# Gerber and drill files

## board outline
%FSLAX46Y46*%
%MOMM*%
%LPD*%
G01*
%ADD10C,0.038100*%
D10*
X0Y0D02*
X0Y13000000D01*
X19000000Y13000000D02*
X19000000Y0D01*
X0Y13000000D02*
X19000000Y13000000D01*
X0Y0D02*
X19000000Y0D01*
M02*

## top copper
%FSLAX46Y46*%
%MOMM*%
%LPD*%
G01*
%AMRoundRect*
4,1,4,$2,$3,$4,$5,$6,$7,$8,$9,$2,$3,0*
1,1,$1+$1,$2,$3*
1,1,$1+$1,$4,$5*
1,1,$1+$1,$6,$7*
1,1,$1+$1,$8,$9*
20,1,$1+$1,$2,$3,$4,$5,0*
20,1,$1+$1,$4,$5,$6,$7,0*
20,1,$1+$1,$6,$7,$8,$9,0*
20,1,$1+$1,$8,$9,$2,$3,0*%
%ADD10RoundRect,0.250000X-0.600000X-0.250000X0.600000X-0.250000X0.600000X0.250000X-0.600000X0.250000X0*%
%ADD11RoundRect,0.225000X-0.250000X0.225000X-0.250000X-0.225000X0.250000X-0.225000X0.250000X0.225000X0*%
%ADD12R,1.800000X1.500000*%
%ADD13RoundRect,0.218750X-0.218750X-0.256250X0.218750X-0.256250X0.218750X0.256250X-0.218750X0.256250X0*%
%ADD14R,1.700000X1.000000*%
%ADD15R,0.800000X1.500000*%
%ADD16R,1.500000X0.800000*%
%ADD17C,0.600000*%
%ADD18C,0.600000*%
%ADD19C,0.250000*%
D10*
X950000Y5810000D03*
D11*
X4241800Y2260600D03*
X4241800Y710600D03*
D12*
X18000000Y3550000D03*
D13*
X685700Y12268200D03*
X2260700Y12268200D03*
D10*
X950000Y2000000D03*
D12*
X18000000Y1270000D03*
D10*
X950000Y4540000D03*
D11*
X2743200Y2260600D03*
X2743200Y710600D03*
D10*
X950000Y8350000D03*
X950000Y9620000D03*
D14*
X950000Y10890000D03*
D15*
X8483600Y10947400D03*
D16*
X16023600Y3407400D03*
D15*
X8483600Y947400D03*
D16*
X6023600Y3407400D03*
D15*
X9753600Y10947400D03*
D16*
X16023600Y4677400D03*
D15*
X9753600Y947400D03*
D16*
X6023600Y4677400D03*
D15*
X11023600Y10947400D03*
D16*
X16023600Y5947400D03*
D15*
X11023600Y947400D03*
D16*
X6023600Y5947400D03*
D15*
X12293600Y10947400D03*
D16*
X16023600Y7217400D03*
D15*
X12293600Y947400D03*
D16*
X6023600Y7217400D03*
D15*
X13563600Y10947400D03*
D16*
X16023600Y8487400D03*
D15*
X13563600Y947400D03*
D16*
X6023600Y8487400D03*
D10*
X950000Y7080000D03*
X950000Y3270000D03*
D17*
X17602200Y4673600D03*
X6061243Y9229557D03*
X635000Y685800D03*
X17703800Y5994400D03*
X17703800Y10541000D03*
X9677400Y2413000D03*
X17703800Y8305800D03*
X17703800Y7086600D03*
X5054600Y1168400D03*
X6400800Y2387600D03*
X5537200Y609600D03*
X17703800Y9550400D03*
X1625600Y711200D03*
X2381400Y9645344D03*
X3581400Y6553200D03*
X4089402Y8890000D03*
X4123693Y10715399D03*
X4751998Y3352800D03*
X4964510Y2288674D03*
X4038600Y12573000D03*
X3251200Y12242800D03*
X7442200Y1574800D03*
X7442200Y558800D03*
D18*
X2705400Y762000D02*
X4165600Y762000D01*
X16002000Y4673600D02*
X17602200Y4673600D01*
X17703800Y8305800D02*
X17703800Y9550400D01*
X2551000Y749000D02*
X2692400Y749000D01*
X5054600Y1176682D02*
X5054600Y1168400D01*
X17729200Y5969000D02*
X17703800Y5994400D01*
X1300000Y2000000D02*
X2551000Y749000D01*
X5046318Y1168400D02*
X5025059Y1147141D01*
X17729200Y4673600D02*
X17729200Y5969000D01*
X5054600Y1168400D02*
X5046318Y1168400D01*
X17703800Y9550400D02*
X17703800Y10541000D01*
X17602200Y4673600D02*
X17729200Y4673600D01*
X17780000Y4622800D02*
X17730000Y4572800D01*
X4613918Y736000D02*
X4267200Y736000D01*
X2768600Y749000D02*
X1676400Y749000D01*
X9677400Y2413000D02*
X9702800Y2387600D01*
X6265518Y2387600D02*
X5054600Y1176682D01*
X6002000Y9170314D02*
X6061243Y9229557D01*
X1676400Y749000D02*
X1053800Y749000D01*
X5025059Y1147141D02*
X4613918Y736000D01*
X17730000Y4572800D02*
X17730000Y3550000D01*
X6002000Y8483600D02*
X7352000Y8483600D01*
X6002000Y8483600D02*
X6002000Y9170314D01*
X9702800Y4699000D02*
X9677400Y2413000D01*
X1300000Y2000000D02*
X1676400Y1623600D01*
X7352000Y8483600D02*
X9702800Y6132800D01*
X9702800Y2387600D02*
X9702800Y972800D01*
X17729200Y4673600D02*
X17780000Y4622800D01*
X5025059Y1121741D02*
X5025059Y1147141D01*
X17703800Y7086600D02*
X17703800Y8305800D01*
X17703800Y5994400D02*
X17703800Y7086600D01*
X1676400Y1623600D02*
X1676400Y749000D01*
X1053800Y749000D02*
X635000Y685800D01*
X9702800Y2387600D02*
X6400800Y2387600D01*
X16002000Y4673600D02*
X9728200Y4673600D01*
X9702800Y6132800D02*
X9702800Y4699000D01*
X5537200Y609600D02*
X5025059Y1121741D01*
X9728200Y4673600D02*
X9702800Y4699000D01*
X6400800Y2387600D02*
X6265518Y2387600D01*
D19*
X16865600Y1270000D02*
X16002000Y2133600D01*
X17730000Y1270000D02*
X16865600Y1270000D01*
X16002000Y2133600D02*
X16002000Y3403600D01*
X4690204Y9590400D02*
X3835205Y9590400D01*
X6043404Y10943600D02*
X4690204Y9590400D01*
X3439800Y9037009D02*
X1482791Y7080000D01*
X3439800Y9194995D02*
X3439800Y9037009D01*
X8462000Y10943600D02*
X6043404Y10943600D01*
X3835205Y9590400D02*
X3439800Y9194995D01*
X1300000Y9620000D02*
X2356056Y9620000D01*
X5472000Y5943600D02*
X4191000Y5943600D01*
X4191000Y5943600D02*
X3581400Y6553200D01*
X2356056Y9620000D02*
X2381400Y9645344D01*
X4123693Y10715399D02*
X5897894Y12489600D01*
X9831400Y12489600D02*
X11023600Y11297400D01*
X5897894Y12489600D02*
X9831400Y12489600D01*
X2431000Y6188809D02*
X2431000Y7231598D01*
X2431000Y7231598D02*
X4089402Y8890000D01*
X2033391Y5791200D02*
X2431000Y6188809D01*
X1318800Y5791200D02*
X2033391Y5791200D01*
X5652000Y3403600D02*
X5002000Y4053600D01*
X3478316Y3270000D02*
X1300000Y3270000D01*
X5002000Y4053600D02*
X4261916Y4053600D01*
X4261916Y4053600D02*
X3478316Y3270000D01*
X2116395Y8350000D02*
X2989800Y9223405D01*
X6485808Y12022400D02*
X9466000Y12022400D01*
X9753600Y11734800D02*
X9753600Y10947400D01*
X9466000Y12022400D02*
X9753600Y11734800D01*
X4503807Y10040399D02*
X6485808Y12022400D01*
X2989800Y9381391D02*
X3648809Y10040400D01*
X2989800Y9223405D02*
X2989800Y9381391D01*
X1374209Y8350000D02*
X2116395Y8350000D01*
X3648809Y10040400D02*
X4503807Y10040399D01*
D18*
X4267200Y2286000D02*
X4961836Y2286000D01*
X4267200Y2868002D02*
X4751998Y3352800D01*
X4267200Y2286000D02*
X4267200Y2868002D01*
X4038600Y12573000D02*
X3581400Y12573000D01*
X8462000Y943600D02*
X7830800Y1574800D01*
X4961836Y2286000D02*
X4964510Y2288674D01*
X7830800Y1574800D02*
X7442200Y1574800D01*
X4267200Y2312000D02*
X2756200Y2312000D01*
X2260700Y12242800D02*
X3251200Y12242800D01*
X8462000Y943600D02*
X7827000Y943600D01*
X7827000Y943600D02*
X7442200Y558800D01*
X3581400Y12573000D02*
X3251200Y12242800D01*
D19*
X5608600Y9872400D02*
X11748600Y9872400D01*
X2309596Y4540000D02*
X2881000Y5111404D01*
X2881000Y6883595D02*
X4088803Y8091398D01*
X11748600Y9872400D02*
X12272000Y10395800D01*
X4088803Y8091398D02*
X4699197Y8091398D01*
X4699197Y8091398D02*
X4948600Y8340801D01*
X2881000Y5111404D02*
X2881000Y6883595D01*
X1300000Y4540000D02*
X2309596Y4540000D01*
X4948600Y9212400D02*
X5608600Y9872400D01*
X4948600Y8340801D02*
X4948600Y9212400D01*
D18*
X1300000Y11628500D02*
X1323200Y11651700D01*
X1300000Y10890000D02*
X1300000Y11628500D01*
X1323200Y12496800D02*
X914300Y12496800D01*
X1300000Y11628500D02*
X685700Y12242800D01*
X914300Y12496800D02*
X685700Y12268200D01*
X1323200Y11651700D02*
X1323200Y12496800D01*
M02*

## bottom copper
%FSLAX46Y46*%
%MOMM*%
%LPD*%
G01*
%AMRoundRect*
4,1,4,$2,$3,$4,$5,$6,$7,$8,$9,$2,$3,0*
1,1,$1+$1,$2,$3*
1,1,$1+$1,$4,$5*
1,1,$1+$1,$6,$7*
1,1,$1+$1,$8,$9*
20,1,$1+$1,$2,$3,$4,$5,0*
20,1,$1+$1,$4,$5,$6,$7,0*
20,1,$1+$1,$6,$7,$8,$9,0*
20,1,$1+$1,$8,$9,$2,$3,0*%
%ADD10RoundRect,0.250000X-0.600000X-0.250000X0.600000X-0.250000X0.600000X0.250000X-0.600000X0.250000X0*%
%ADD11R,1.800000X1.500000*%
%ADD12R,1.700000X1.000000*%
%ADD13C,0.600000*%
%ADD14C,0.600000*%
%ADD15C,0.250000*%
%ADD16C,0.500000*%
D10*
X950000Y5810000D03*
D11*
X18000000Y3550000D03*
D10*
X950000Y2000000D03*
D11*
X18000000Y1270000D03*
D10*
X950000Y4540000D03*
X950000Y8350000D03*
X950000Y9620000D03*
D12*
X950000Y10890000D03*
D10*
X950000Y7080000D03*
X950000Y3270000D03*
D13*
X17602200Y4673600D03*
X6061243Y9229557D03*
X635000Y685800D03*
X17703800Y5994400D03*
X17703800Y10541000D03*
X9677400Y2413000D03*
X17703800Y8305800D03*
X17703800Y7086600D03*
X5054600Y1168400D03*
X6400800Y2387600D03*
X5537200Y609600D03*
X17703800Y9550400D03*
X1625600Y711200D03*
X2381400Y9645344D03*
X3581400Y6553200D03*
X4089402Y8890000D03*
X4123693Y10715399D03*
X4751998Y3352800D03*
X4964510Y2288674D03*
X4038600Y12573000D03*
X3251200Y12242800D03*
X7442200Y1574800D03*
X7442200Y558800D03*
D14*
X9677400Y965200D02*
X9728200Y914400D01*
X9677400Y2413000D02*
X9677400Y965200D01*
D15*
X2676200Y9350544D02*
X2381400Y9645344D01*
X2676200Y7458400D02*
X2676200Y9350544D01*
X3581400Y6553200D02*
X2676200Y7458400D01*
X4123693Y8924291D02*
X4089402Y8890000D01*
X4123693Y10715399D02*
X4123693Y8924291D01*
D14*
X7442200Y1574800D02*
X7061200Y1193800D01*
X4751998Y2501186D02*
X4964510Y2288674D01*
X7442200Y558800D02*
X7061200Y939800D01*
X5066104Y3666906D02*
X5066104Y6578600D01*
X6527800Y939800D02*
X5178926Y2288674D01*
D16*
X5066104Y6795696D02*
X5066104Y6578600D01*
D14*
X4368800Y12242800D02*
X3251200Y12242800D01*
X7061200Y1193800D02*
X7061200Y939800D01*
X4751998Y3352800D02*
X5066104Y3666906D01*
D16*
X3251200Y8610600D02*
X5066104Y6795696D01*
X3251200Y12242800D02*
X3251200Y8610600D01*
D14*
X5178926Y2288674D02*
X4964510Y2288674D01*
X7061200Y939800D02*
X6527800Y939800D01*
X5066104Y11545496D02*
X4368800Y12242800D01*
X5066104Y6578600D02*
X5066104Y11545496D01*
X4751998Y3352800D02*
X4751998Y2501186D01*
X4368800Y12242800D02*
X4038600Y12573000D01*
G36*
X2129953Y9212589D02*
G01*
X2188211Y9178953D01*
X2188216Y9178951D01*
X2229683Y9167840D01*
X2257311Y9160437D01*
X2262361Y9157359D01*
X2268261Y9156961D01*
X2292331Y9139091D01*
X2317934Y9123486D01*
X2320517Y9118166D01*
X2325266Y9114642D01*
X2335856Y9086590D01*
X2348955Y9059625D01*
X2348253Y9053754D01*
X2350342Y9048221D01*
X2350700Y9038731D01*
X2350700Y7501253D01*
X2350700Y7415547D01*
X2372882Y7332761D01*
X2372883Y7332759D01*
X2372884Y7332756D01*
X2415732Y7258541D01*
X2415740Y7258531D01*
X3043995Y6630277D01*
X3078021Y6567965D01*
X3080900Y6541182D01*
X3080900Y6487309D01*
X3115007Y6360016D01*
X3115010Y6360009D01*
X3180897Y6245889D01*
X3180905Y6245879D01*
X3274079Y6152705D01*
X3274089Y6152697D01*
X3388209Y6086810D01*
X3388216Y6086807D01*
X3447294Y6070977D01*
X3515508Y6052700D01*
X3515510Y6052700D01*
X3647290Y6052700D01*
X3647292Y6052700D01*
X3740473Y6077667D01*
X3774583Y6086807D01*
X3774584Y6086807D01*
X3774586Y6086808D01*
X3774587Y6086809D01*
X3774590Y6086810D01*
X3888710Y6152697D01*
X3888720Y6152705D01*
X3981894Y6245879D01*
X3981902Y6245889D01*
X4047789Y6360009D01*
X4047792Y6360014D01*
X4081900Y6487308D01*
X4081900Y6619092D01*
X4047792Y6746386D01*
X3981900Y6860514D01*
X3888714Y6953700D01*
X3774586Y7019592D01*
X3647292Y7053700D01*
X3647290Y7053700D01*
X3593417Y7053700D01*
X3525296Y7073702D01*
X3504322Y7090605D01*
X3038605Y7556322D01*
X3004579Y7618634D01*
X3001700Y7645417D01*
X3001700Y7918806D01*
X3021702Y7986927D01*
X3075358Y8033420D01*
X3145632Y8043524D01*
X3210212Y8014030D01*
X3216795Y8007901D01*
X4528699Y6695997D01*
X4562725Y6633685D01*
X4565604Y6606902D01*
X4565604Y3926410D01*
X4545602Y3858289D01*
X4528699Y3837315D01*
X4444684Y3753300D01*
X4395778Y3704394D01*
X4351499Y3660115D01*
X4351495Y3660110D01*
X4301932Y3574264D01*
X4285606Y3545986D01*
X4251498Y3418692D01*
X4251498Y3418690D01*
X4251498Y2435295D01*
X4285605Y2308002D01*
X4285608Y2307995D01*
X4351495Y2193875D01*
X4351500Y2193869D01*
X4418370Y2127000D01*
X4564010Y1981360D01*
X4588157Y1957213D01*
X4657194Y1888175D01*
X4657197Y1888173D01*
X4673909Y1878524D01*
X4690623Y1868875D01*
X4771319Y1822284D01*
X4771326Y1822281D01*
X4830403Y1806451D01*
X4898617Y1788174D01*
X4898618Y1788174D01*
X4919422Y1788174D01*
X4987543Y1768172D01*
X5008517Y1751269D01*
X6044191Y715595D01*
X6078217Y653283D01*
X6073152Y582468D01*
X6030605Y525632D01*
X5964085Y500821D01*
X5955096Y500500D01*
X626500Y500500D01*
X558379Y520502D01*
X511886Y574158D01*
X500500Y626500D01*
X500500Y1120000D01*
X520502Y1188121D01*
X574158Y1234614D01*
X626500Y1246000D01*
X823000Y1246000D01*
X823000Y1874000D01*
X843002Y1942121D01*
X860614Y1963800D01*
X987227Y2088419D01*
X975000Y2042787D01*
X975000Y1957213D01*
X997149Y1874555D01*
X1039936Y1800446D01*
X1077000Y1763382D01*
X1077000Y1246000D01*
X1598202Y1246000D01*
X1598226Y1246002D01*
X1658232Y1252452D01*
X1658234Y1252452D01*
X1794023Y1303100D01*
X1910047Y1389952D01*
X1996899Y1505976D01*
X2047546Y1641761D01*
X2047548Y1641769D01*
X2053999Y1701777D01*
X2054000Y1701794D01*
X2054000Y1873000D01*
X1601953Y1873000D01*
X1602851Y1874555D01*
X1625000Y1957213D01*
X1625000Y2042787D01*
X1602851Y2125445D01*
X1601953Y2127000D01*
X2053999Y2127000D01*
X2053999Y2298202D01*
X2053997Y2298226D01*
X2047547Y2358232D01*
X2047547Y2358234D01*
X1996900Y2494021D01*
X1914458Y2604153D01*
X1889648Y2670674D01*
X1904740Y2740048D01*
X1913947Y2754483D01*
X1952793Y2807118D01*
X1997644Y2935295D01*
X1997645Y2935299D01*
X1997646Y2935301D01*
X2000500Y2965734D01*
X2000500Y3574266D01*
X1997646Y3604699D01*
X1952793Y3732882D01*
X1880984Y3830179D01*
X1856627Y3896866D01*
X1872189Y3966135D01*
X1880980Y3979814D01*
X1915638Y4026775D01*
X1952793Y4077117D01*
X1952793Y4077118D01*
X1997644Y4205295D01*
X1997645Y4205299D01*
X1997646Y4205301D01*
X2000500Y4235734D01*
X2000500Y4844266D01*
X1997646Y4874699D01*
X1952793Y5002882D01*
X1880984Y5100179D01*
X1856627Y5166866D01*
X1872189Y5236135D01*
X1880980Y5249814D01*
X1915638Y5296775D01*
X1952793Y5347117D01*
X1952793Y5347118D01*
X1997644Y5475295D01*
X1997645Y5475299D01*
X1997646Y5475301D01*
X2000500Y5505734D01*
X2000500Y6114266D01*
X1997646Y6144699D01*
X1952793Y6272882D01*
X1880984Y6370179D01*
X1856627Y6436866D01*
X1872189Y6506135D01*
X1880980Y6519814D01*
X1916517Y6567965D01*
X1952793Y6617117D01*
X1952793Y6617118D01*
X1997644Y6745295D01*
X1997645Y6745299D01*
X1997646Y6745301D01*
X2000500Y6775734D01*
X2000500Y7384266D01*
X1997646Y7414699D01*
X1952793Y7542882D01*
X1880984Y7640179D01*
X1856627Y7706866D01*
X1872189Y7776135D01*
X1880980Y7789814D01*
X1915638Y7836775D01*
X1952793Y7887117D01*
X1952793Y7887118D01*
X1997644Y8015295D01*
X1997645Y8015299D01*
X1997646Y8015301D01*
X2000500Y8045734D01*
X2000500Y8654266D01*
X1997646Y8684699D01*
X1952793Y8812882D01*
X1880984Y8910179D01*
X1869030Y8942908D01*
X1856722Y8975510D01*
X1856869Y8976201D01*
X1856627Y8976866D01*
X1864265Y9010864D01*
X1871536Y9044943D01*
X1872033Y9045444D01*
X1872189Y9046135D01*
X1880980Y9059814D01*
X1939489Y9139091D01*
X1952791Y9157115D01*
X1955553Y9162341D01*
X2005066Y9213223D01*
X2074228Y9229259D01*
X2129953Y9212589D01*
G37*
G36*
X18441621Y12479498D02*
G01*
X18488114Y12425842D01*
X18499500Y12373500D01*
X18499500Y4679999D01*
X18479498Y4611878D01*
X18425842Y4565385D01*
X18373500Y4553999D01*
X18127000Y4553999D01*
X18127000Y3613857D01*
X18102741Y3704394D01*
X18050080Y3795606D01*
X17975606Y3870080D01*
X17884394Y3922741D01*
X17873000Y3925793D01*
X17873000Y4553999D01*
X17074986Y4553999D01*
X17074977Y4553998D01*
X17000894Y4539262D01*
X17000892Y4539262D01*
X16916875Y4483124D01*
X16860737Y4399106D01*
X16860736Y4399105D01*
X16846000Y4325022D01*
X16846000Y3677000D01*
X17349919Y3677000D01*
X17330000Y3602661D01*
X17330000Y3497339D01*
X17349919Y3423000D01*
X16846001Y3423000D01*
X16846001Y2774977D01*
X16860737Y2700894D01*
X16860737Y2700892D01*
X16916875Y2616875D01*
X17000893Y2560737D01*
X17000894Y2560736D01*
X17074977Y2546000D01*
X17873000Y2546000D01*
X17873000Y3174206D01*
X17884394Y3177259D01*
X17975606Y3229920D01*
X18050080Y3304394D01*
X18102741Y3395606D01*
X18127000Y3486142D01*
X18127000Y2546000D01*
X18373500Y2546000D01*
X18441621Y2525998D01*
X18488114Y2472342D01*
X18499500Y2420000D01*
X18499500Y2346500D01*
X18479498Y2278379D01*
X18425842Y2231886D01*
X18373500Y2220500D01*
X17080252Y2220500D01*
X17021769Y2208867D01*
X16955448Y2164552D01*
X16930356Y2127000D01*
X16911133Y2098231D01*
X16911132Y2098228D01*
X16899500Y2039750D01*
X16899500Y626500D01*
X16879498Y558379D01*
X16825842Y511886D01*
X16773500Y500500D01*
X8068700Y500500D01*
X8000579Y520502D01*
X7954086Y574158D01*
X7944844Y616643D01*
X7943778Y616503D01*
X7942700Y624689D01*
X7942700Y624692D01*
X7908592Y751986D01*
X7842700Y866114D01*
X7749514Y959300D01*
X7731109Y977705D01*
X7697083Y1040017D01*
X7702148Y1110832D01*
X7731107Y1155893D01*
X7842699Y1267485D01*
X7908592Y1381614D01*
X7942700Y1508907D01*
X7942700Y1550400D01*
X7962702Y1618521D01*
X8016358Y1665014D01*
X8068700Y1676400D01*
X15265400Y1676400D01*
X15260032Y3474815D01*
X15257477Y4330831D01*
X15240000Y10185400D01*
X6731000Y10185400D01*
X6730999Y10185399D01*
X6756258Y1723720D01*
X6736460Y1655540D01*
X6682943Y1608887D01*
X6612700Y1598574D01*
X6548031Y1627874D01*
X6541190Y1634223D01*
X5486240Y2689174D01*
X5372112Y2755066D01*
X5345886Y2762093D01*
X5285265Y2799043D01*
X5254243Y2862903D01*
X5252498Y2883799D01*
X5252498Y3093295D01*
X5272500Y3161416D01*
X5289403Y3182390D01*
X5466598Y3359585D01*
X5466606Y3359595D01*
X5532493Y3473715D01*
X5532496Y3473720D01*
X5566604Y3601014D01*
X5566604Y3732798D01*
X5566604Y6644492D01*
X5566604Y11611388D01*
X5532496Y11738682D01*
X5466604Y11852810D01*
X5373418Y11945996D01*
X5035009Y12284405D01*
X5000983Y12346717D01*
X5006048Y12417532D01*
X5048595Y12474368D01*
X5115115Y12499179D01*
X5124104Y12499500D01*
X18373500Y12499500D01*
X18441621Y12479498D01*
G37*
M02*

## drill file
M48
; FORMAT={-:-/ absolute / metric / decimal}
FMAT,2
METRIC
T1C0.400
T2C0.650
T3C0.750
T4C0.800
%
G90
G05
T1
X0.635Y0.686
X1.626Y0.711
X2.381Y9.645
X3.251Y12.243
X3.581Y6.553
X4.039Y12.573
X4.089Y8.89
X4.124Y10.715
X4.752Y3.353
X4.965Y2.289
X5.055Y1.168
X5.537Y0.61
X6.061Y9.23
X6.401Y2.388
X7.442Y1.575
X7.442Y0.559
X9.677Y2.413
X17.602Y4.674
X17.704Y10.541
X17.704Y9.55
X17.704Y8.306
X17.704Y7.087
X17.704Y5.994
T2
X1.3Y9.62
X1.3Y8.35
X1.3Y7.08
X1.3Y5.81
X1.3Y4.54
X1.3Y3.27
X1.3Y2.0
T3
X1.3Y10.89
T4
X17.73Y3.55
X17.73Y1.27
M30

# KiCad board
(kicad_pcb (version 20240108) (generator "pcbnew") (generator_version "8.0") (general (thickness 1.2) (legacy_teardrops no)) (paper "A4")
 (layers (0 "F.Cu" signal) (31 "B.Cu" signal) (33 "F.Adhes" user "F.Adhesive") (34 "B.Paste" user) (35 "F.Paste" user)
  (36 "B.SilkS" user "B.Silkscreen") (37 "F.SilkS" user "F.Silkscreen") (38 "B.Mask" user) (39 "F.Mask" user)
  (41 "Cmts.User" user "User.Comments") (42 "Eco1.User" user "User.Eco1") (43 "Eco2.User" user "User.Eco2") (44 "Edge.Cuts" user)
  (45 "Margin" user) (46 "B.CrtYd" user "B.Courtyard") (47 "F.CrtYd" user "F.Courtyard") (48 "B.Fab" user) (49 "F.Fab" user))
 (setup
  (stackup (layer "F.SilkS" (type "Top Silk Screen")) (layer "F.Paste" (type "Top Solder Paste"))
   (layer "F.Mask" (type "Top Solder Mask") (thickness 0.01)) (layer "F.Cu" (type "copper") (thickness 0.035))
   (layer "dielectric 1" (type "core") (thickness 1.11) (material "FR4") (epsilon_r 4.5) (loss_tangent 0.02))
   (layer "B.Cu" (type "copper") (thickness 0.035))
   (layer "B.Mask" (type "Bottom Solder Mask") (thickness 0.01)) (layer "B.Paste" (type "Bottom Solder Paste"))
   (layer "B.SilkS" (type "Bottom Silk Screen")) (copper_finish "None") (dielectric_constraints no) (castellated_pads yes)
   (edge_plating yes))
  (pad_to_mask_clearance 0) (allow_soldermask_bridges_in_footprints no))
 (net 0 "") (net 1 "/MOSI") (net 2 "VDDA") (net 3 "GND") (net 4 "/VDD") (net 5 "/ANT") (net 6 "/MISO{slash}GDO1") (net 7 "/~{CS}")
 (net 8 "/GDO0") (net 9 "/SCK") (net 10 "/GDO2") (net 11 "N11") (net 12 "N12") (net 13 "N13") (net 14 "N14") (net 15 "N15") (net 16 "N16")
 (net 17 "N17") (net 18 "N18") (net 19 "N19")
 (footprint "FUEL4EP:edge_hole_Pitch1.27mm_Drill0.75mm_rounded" (layer "F.Cu") (at 0 -5.81)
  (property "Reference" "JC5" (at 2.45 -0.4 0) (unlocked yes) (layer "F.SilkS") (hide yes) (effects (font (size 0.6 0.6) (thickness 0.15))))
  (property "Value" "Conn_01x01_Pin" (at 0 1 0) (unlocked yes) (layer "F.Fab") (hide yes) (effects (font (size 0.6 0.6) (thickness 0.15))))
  (pad "1" thru_hole roundrect (at 1.3 0) (size 1.7 1) (drill 0.65 (offset -0.35 0)) (layers "*.Cu" "*.Mask") (remove_unused_layers no)
   (roundrect_rratio 0.25) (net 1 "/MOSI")))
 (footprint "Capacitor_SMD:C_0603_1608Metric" (layer "F.Cu") (at 4.2418 -1.4856 -90)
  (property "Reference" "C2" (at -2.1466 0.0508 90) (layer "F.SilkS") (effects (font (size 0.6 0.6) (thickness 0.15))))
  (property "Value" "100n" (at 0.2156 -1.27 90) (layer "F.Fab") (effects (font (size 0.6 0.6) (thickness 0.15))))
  (pad "1" smd roundrect (at -0.775 0 270) (size 0.9 0.95) (layers "F.Cu" "F.Paste" "F.Mask") (roundrect_rratio 0.25) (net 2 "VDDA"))
  (pad "2" smd roundrect (at 0.775 0 270) (size 0.9 0.95) (layers "F.Cu" "F.Paste" "F.Mask") (roundrect_rratio 0.25) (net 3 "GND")))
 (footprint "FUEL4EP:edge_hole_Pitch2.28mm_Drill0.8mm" (layer "F.Cu") (at 19 -3.55 180)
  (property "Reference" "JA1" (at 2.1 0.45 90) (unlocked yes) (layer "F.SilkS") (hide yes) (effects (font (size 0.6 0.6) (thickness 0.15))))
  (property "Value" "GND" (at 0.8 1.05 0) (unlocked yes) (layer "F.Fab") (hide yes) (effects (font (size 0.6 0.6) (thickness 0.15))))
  (pad "1" thru_hole rect (at 1.27 0 180) (size 1.8 1.5) (drill 0.8 (offset -0.27 0)) (layers "*.Cu" "*.Mask") (remove_unused_layers no)
   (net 3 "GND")))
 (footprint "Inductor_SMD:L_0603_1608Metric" (layer "F.Cu") (at 1.4732 -12.2682)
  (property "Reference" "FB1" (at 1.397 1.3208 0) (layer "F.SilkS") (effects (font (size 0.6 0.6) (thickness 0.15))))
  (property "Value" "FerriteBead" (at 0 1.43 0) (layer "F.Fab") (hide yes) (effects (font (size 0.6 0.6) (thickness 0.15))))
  (pad "1" smd roundrect (at -0.7875 0) (size 0.875 0.95) (layers "F.Cu" "F.Paste" "F.Mask") (roundrect_rratio 0.25) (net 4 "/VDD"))
  (pad "2" smd roundrect (at 0.7875 0) (size 0.875 0.95) (layers "F.Cu" "F.Paste" "F.Mask") (roundrect_rratio 0.25) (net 2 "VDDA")))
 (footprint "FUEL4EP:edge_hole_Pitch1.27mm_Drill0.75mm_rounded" (layer "F.Cu") (at 0 -2)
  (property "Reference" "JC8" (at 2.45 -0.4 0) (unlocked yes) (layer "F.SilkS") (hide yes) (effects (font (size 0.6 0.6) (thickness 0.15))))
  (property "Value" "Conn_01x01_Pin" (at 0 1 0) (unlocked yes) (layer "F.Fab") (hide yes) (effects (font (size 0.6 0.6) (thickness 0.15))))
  (pad "1" thru_hole roundrect (at 1.3 0) (size 1.7 1) (drill 0.65 (offset -0.35 0)) (layers "*.Cu" "*.Mask") (remove_unused_layers no)
   (roundrect_rratio 0.25) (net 3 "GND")))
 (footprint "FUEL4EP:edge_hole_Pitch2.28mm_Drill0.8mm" (layer "F.Cu") (at 19 -1.27 180)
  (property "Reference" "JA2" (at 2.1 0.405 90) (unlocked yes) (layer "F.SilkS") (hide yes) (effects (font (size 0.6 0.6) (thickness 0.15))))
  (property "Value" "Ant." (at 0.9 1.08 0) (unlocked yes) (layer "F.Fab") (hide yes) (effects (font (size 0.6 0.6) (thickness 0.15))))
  (pad "1" thru_hole rect (at 1.27 0 180) (size 1.8 1.5) (drill 0.8 (offset -0.27 0)) (layers "*.Cu" "*.Mask") (remove_unused_layers no)
   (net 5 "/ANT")))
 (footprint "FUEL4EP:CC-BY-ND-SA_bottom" (layer "F.Cu") (at 9.4996 -4.2164 180)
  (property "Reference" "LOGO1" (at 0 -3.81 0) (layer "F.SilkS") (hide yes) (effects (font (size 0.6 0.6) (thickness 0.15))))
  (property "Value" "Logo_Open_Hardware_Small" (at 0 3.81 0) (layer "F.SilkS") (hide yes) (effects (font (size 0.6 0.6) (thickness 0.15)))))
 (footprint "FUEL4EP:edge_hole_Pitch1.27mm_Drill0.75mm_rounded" (layer "F.Cu") (at 0 -4.54)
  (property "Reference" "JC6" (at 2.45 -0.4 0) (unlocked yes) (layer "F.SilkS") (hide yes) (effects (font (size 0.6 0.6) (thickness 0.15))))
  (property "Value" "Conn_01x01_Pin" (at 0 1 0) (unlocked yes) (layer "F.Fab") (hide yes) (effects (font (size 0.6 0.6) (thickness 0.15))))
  (pad "1" thru_hole roundrect (at 1.3 0) (size 1.7 1) (drill 0.65 (offset -0.35 0)) (layers "*.Cu" "*.Mask") (remove_unused_layers no)
   (roundrect_rratio 0.25) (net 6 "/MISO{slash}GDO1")))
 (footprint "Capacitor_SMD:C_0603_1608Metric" (layer "F.Cu") (at 2.7432 -1.4856 -90)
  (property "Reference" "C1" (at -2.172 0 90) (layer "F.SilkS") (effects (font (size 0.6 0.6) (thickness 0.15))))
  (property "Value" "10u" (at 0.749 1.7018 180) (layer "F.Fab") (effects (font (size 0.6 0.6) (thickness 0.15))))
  (pad "1" smd roundrect (at -0.775 0 270) (size 0.9 0.95) (layers "F.Cu" "F.Paste" "F.Mask") (roundrect_rratio 0.25) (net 2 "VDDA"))
  (pad "2" smd roundrect (at 0.775 0 270) (size 0.9 0.95) (layers "F.Cu" "F.Paste" "F.Mask") (roundrect_rratio 0.25) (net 3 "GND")))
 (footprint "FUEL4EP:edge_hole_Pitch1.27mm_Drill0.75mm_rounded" (layer "F.Cu") (at 0 -8.35)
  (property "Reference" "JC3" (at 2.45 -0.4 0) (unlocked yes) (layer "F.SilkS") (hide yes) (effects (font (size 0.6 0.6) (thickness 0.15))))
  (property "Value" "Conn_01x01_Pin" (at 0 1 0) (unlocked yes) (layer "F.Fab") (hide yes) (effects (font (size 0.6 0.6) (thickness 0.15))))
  (pad "1" thru_hole roundrect (at 1.3 0) (size 1.7 1) (drill 0.65 (offset -0.35 0)) (layers "*.Cu" "*.Mask") (remove_unused_layers no)
   (roundrect_rratio 0.25) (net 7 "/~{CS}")))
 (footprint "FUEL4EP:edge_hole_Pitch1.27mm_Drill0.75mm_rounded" (layer "F.Cu") (at 0 -9.62)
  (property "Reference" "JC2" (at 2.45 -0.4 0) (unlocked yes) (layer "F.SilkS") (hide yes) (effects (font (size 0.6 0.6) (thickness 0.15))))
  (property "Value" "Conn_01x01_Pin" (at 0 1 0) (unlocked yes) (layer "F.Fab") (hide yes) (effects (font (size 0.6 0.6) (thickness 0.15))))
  (pad "1" thru_hole roundrect (at 1.3 0) (size 1.7 1) (drill 0.65 (offset -0.35 0)) (layers "*.Cu" "*.Mask") (remove_unused_layers no)
   (roundrect_rratio 0.25) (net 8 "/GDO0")))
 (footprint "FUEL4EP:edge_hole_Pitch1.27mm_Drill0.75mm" (layer "F.Cu") (at 0 -10.89)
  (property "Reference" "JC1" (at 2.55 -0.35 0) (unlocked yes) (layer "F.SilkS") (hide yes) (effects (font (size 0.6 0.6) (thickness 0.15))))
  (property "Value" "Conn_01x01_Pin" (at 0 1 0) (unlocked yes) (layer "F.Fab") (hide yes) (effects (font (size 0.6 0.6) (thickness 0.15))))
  (pad "1" thru_hole rect (at 1.3 0) (size 1.7 1) (drill 0.75 (offset -0.35 0)) (layers "*.Cu" "*.Mask") (remove_unused_layers no)
   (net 4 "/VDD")))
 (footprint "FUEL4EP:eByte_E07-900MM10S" (layer "F.Cu") (at 6.0236 -0.9474 90)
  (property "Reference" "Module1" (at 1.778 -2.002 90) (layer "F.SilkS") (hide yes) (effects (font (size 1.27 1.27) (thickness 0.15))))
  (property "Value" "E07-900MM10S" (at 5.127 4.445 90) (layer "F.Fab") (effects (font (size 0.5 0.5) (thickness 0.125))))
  (pad "1A" smd rect (at 10 2.46 270) (size 1.5 0.8) (layers "F.Cu" "F.Paste" "F.Mask") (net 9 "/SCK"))
  (pad "1B" smd rect (at 2.46 10 180) (size 1.5 0.8) (layers "F.Cu" "F.Paste" "F.Mask") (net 5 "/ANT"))
  (pad "1C" smd rect (at 0 2.46 90) (size 1.5 0.8) (layers "F.Cu" "F.Paste" "F.Mask") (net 2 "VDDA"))
  (pad "1D" smd rect (at 2.46 0) (size 1.5 0.8) (layers "F.Cu" "F.Paste" "F.Mask") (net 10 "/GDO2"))
  (pad "2A" smd rect (at 10 3.73 270) (size 1.5 0.8) (layers "F.Cu" "F.Paste" "F.Mask") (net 7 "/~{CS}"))
  (pad "2B" smd rect (at 3.73 10 180) (size 1.5 0.8) (layers "F.Cu" "F.Paste" "F.Mask") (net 3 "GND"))
  (pad "2C" smd rect (at 0 3.73 90) (size 1.5 0.8) (layers "F.Cu" "F.Paste" "F.Mask") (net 3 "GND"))
  (pad "2D" smd rect (at 3.73 0) (size 1.5 0.8) (layers "F.Cu" "F.Paste" "F.Mask") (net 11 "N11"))
  (pad "3A" smd rect (at 10 5 270) (size 1.5 0.8) (layers "F.Cu" "F.Paste" "F.Mask") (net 1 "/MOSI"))
  (pad "3B" smd rect (at 5 10 180) (size 1.5 0.8) (layers "F.Cu" "F.Paste" "F.Mask") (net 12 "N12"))
  (pad "3C" smd rect (at 0 5 90) (size 1.5 0.8) (layers "F.Cu" "F.Paste" "F.Mask") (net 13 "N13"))
  (pad "3D" smd rect (at 5 0) (size 1.5 0.8) (layers "F.Cu" "F.Paste" "F.Mask") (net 8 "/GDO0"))
  (pad "4A" smd rect (at 10 6.27 270) (size 1.5 0.8) (layers "F.Cu" "F.Paste" "F.Mask") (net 6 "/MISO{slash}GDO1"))
  (pad "4B" smd rect (at 6.27 10 180) (size 1.5 0.8) (layers "F.Cu" "F.Paste" "F.Mask") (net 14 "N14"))
  (pad "4C" smd rect (at 0 6.27 90) (size 1.5 0.8) (layers "F.Cu" "F.Paste" "F.Mask") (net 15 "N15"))
  (pad "4D" smd rect (at 6.27 0) (size 1.5 0.8) (layers "F.Cu" "F.Paste" "F.Mask") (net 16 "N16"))
  (pad "5A" smd rect (at 10 7.54 270) (size 1.5 0.8) (layers "F.Cu" "F.Paste" "F.Mask") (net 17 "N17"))
  (pad "5B" smd rect (at 7.54 10 180) (size 1.5 0.8) (layers "F.Cu" "F.Paste" "F.Mask") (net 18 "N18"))
  (pad "5C" smd rect (at 0 7.54 90) (size 1.5 0.8) (layers "F.Cu" "F.Paste" "F.Mask") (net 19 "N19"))
  (pad "5D" smd rect (at 7.54 0) (size 1.5 0.8) (layers "F.Cu" "F.Paste" "F.Mask") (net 3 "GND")))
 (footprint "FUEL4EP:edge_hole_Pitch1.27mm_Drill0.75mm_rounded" (layer "F.Cu") (at 0 -7.08)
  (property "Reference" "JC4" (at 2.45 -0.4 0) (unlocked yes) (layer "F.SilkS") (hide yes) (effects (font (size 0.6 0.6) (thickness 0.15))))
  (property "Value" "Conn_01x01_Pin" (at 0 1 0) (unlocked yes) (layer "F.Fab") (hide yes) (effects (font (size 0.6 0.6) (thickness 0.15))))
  (pad "1" thru_hole roundrect (at 1.3 0) (size 1.7 1) (drill 0.65 (offset -0.35 0)) (layers "*.Cu" "*.Mask") (remove_unused_layers no)
   (roundrect_rratio 0.25) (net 9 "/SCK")))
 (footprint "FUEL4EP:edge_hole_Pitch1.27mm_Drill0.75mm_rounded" (layer "F.Cu") (at 0 -3.27)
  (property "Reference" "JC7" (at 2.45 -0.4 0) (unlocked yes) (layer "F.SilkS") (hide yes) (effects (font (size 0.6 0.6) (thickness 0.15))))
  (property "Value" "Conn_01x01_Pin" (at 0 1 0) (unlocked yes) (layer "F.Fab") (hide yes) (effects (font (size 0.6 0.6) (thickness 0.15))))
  (pad "1" thru_hole roundrect (at 1.3 0) (size 1.7 1) (drill 0.65 (offset -0.35 0)) (layers "*.Cu" "*.Mask") (remove_unused_layers no)
   (roundrect_rratio 0.25) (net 10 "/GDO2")))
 (gr_line (start 0 0) (end 0 -13) (stroke (width 0.0381) (type solid)) (layer "Edge.Cuts"))
 (gr_line (start 19 -13) (end 19 0) (stroke (width 0.0381) (type solid)) (layer "Edge.Cuts"))
 (gr_line (start 0 -13) (end 19 -13) (stroke (width 0.0381) (type solid)) (layer "Edge.Cuts"))
 (gr_line (start 0 0) (end 19 0) (stroke (width 0.0381) (type solid)) (layer "Edge.Cuts"))
 (segment (start 2.7054 -0.762) (end 4.1656 -0.762) (width 0.6) (layer "F.Cu") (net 3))
 (segment (start 16.002 -4.6736) (end 17.6022 -4.6736) (width 0.6) (layer "F.Cu") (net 3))
 (segment (start 17.7038 -8.3058) (end 17.7038 -9.5504) (width 0.6) (layer "F.Cu") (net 3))
 (segment (start 2.551 -0.749) (end 2.6924 -0.749) (width 0.6) (layer "F.Cu") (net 3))
 (segment (start 5.0546 -1.176682) (end 5.0546 -1.1684) (width 0.6) (layer "F.Cu") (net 3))
 (segment (start 17.7292 -5.969) (end 17.7038 -5.9944) (width 0.6) (layer "F.Cu") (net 3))
 (segment (start 1.3 -2) (end 2.551 -0.749) (width 0.6) (layer "F.Cu") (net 3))
 (segment (start 5.046318 -1.1684) (end 5.025059 -1.147141) (width 0.6) (layer "F.Cu") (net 3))
 (segment (start 17.7292 -4.6736) (end 17.7292 -5.969) (width 0.6) (layer "F.Cu") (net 3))
 (segment (start 5.0546 -1.1684) (end 5.046318 -1.1684) (width 0.6) (layer "F.Cu") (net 3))
 (segment (start 17.7038 -9.5504) (end 17.7038 -10.541) (width 0.6) (layer "F.Cu") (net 3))
 (segment (start 17.6022 -4.6736) (end 17.7292 -4.6736) (width 0.6) (layer "F.Cu") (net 3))
 (segment (start 17.78 -4.6228) (end 17.73 -4.5728) (width 0.6) (layer "F.Cu") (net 3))
 (segment (start 4.613918 -0.736) (end 4.2672 -0.736) (width 0.6) (layer "F.Cu") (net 3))
 (segment (start 2.7686 -0.749) (end 1.6764 -0.749) (width 0.6) (layer "F.Cu") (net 3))
 (segment (start 9.6774 -2.413) (end 9.7028 -2.3876) (width 0.6) (layer "F.Cu") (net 3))
 (segment (start 6.265518 -2.3876) (end 5.0546 -1.176682) (width 0.6) (layer "F.Cu") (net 3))
 (segment (start 6.002 -9.170314) (end 6.061243 -9.229557) (width 0.6) (layer "F.Cu") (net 3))
 (segment (start 1.6764 -0.749) (end 1.0538 -0.749) (width 0.6) (layer "F.Cu") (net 3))
 (segment (start 5.025059 -1.147141) (end 4.613918 -0.736) (width 0.6) (layer "F.Cu") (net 3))
 (segment (start 17.73 -4.5728) (end 17.73 -3.55) (width 0.6) (layer "F.Cu") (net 3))
 (segment (start 6.002 -8.4836) (end 7.352 -8.4836) (width 0.6) (layer "F.Cu") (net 3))
 (segment (start 6.002 -8.4836) (end 6.002 -9.170314) (width 0.6) (layer "F.Cu") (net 3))
 (segment (start 9.7028 -4.699) (end 9.6774 -2.413) (width 0.6) (layer "F.Cu") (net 3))
 (segment (start 1.3 -2) (end 1.6764 -1.6236) (width 0.6) (layer "F.Cu") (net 3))
 (segment (start 7.352 -8.4836) (end 9.7028 -6.1328) (width 0.6) (layer "F.Cu") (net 3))
 (segment (start 9.7028 -2.3876) (end 9.7028 -0.9728) (width 0.6) (layer "F.Cu") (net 3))
 (segment (start 17.7292 -4.6736) (end 17.78 -4.6228) (width 0.6) (layer "F.Cu") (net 3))
 (segment (start 5.025059 -1.121741) (end 5.025059 -1.147141) (width 0.6) (layer "F.Cu") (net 3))
 (segment (start 17.7038 -7.0866) (end 17.7038 -8.3058) (width 0.6) (layer "F.Cu") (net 3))
 (segment (start 17.7038 -5.9944) (end 17.7038 -7.0866) (width 0.6) (layer "F.Cu") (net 3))
 (segment (start 1.6764 -1.6236) (end 1.6764 -0.749) (width 0.6) (layer "F.Cu") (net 3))
 (segment (start 1.0538 -0.749) (end 0.635 -0.6858) (width 0.6) (layer "F.Cu") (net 3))
 (segment (start 9.7028 -2.3876) (end 6.4008 -2.3876) (width 0.6) (layer "F.Cu") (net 3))
 (segment (start 16.002 -4.6736) (end 9.7282 -4.6736) (width 0.6) (layer "F.Cu") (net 3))
 (segment (start 9.7028 -6.1328) (end 9.7028 -4.699) (width 0.6) (layer "F.Cu") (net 3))
 (segment (start 5.5372 -0.6096) (end 5.025059 -1.121741) (width 0.6) (layer "F.Cu") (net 3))
 (segment (start 9.7282 -4.6736) (end 9.7028 -4.699) (width 0.6) (layer "F.Cu") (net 3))
 (segment (start 6.4008 -2.3876) (end 6.265518 -2.3876) (width 0.6) (layer "F.Cu") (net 3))
 (via (at 17.6022 -4.6736) (size 0.6) (drill 0.4) (layers "F.Cu" "B.Cu") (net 3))
 (via (at 6.061243 -9.229557) (size 0.6) (drill 0.4) (layers "F.Cu" "B.Cu") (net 3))
 (via (at 0.635 -0.6858) (size 0.6) (drill 0.4) (layers "F.Cu" "B.Cu") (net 3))
 (via (at 17.7038 -5.9944) (size 0.6) (drill 0.4) (layers "F.Cu" "B.Cu") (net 3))
 (via (at 17.7038 -10.541) (size 0.6) (drill 0.4) (layers "F.Cu" "B.Cu") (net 3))
 (via (at 9.6774 -2.413) (size 0.6) (drill 0.4) (layers "F.Cu" "B.Cu") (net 3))
 (via (at 17.7038 -8.3058) (size 0.6) (drill 0.4) (layers "F.Cu" "B.Cu") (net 3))
 (via (at 17.7038 -7.0866) (size 0.6) (drill 0.4) (layers "F.Cu" "B.Cu") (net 3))
 (via (at 5.0546 -1.1684) (size 0.6) (drill 0.4) (layers "F.Cu" "B.Cu") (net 3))
 (via (at 6.4008 -2.3876) (size 0.6) (drill 0.4) (layers "F.Cu" "B.Cu") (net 3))
 (via (at 5.5372 -0.6096) (size 0.6) (drill 0.4) (layers "F.Cu" "B.Cu") (free yes) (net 3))
 (via (at 17.7038 -9.5504) (size 0.6) (drill 0.4) (layers "F.Cu" "B.Cu") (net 3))
 (via (at 1.6256 -0.7112) (size 0.6) (drill 0.4) (layers "F.Cu" "B.Cu") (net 3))
 (segment (start 9.6774 -0.9652) (end 9.7282 -0.9144) (width 0.6) (layer "B.Cu") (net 3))
 (segment (start 9.6774 -2.413) (end 9.6774 -0.9652) (width 0.6) (layer "B.Cu") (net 3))
 (segment (start 16.8656 -1.27) (end 16.002 -2.1336) (width 0.25) (layer "F.Cu") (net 5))
 (segment (start 17.73 -1.27) (end 16.8656 -1.27) (width 0.25) (layer "F.Cu") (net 5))
 (segment (start 16.002 -2.1336) (end 16.002 -3.4036) (width 0.25) (layer "F.Cu") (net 5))
 (segment (start 4.690204 -9.5904) (end 3.835205 -9.5904) (width 0.25) (layer "F.Cu") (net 9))
 (segment (start 6.043404 -10.9436) (end 4.690204 -9.5904) (width 0.25) (layer "F.Cu") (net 9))
 (segment (start 3.4398 -9.037009) (end 1.482791 -7.08) (width 0.25) (layer "F.Cu") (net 9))
 (segment (start 3.4398 -9.194995) (end 3.4398 -9.037009) (width 0.25) (layer "F.Cu") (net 9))
 (segment (start 8.462 -10.9436) (end 6.043404 -10.9436) (width 0.25) (layer "F.Cu") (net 9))
 (segment (start 3.835205 -9.5904) (end 3.4398 -9.194995) (width 0.25) (layer "F.Cu") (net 9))
 (segment (start 1.3 -9.62) (end 2.356056 -9.62) (width 0.25) (layer "F.Cu") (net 8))
 (segment (start 5.472 -5.9436) (end 4.191 -5.9436) (width 0.25) (layer "F.Cu") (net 8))
 (segment (start 4.191 -5.9436) (end 3.5814 -6.5532) (width 0.25) (layer "F.Cu") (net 8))
 (segment (start 2.356056 -9.62) (end 2.3814 -9.645344) (width 0.25) (layer "F.Cu") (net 8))
 (via (at 2.3814 -9.645344) (size 0.6) (drill 0.4) (layers "F.Cu" "B.Cu") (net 8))
 (via (at 3.5814 -6.5532) (size 0.6) (drill 0.4) (layers "F.Cu" "B.Cu") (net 8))
 (segment (start 2.6762 -9.350544) (end 2.3814 -9.645344) (width 0.25) (layer "B.Cu") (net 8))
 (segment (start 2.6762 -7.4584) (end 2.6762 -9.350544) (width 0.25) (layer "B.Cu") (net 8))
 (segment (start 3.5814 -6.5532) (end 2.6762 -7.4584) (width 0.25) (layer "B.Cu") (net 8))
 (segment (start 4.123693 -10.715399) (end 5.897894 -12.4896) (width 0.25) (layer "F.Cu") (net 1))
 (segment (start 9.8314 -12.4896) (end 11.0236 -11.2974) (width 0.25) (layer "F.Cu") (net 1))
 (segment (start 5.897894 -12.4896) (end 9.8314 -12.4896) (width 0.25) (layer "F.Cu") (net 1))
 (segment (start 2.431 -6.188809) (end 2.431 -7.231598) (width 0.25) (layer "F.Cu") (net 1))
 (segment (start 2.431 -7.231598) (end 4.089402 -8.89) (width 0.25) (layer "F.Cu") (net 1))
 (segment (start 2.033391 -5.7912) (end 2.431 -6.188809) (width 0.25) (layer "F.Cu") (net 1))
 (segment (start 1.3188 -5.7912) (end 2.033391 -5.7912) (width 0.25) (layer "F.Cu") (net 1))
 (via (at 4.089402 -8.89) (size 0.6) (drill 0.4) (layers "F.Cu" "B.Cu") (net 1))
 (via (at 4.123693 -10.715399) (size 0.6) (drill 0.4) (layers "F.Cu" "B.Cu") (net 1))
 (segment (start 4.123693 -8.924291) (end 4.089402 -8.89) (width 0.25) (layer "B.Cu") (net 1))
 (segment (start 4.123693 -10.715399) (end 4.123693 -8.924291) (width 0.25) (layer "B.Cu") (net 1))
 (segment (start 5.652 -3.4036) (end 5.002 -4.0536) (width 0.25) (layer "F.Cu") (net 10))
 (segment (start 3.478316 -3.27) (end 1.3 -3.27) (width 0.25) (layer "F.Cu") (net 10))
 (segment (start 5.002 -4.0536) (end 4.261916 -4.0536) (width 0.25) (layer "F.Cu") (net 10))
 (segment (start 4.261916 -4.0536) (end 3.478316 -3.27) (width 0.25) (layer "F.Cu") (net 10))
 (segment (start 2.116395 -8.35) (end 2.9898 -9.223405) (width 0.25) (layer "F.Cu") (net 7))
 (segment (start 6.485808 -12.0224) (end 9.466 -12.0224) (width 0.25) (layer "F.Cu") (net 7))
 (segment (start 9.7536 -11.7348) (end 9.7536 -10.9474) (width 0.25) (layer "F.Cu") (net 7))
 (segment (start 9.466 -12.0224) (end 9.7536 -11.7348) (width 0.25) (layer "F.Cu") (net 7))
 (segment (start 4.503807 -10.040399) (end 6.485808 -12.0224) (width 0.25) (layer "F.Cu") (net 7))
 (segment (start 2.9898 -9.381391) (end 3.648809 -10.0404) (width 0.25) (layer "F.Cu") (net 7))
 (segment (start 2.9898 -9.223405) (end 2.9898 -9.381391) (width 0.25) (layer "F.Cu") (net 7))
 (segment (start 1.374209 -8.35) (end 2.116395 -8.35) (width 0.25) (layer "F.Cu") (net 7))
 (segment (start 3.648809 -10.0404) (end 4.503807 -10.040399) (width 0.25) (layer "F.Cu") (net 7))
 (segment (start 4.2672 -2.286) (end 4.961836 -2.286) (width 0.6) (layer "F.Cu") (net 2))
 (segment (start 4.2672 -2.868002) (end 4.751998 -3.3528) (width 0.6) (layer "F.Cu") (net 2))
 (segment (start 4.2672 -2.286) (end 4.2672 -2.868002) (width 0.6) (layer "F.Cu") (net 2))
 (segment (start 4.0386 -12.573) (end 3.5814 -12.573) (width 0.6) (layer "F.Cu") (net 2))
 (segment (start 8.462 -0.9436) (end 7.8308 -1.5748) (width 0.6) (layer "F.Cu") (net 2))
 (segment (start 4.961836 -2.286) (end 4.96451 -2.288674) (width 0.6) (layer "F.Cu") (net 2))
 (segment (start 7.8308 -1.5748) (end 7.4422 -1.5748) (width 0.6) (layer "F.Cu") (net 2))
 (segment (start 4.2672 -2.312) (end 2.7562 -2.312) (width 0.6) (layer "F.Cu") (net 2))
 (segment (start 2.2607 -12.2428) (end 3.2512 -12.2428) (width 0.6) (layer "F.Cu") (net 2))
 (segment (start 8.462 -0.9436) (end 7.827 -0.9436) (width 0.6) (layer "F.Cu") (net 2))
 (segment (start 7.827 -0.9436) (end 7.4422 -0.5588) (width 0.6) (layer "F.Cu") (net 2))
 (segment (start 3.5814 -12.573) (end 3.2512 -12.2428) (width 0.6) (layer "F.Cu") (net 2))
 (via (at 4.751998 -3.3528) (size 0.6) (drill 0.4) (layers "F.Cu" "B.Cu") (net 2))
 (via (at 4.96451 -2.288674) (size 0.6) (drill 0.4) (layers "F.Cu" "B.Cu") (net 2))
 (via (at 4.0386 -12.573) (size 0.6) (drill 0.4) (layers "F.Cu" "B.Cu") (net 2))
 (via (at 3.2512 -12.2428) (size 0.6) (drill 0.4) (layers "F.Cu" "B.Cu") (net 2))
 (via (at 7.4422 -1.5748) (size 0.6) (drill 0.4) (layers "F.Cu" "B.Cu") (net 2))
 (via (at 7.4422 -0.5588) (size 0.6) (drill 0.4) (layers "F.Cu" "B.Cu") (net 2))
 (segment (start 7.4422 -1.5748) (end 7.0612 -1.1938) (width 0.6) (layer "B.Cu") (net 2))
 (segment (start 4.751998 -2.501186) (end 4.96451 -2.288674) (width 0.6) (layer "B.Cu") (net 2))
 (segment (start 7.4422 -0.5588) (end 7.0612 -0.9398) (width 0.6) (layer "B.Cu") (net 2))
 (segment (start 5.066104 -3.666906) (end 5.066104 -6.5786) (width 0.6) (layer "B.Cu") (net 2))
 (segment (start 6.5278 -0.9398) (end 5.178926 -2.288674) (width 0.6) (layer "B.Cu") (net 2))
 (segment (start 5.066104 -6.795696) (end 5.066104 -6.5786) (width 0.5) (layer "B.Cu") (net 2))
 (segment (start 4.3688 -12.2428) (end 3.2512 -12.2428) (width 0.6) (layer "B.Cu") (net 2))
 (segment (start 7.0612 -1.1938) (end 7.0612 -0.9398) (width 0.6) (layer "B.Cu") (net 2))
 (segment (start 4.751998 -3.3528) (end 5.066104 -3.666906) (width 0.6) (layer "B.Cu") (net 2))
 (segment (start 3.2512 -8.6106) (end 5.066104 -6.795696) (width 0.5) (layer "B.Cu") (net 2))
 (segment (start 3.2512 -12.2428) (end 3.2512 -8.6106) (width 0.5) (layer "B.Cu") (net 2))
 (segment (start 5.178926 -2.288674) (end 4.96451 -2.288674) (width 0.6) (layer "B.Cu") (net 2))
 (segment (start 7.0612 -0.9398) (end 6.5278 -0.9398) (width 0.6) (layer "B.Cu") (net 2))
 (segment (start 5.066104 -11.545496) (end 4.3688 -12.2428) (width 0.6) (layer "B.Cu") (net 2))
 (segment (start 5.066104 -6.5786) (end 5.066104 -11.545496) (width 0.6) (layer "B.Cu") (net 2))
 (segment (start 4.751998 -3.3528) (end 4.751998 -2.501186) (width 0.6) (layer "B.Cu") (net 2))
 (segment (start 4.3688 -12.2428) (end 4.0386 -12.573) (width 0.6) (layer "B.Cu") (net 2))
 (segment (start 5.6086 -9.8724) (end 11.7486 -9.8724) (width 0.25) (layer "F.Cu") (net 6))
 (segment (start 2.309596 -4.54) (end 2.881 -5.111404) (width 0.25) (layer "F.Cu") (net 6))
 (segment (start 2.881 -6.883595) (end 4.088803 -8.091398) (width 0.25) (layer "F.Cu") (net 6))
 (segment (start 11.7486 -9.8724) (end 12.272 -10.3958) (width 0.25) (layer "F.Cu") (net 6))
 (segment (start 4.088803 -8.091398) (end 4.699197 -8.091398) (width 0.25) (layer "F.Cu") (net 6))
 (segment (start 4.699197 -8.091398) (end 4.9486 -8.340801) (width 0.25) (layer "F.Cu") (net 6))
 (segment (start 2.881 -5.111404) (end 2.881 -6.883595) (width 0.25) (layer "F.Cu") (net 6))
 (segment (start 1.3 -4.54) (end 2.309596 -4.54) (width 0.25) (layer "F.Cu") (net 6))
 (segment (start 4.9486 -9.2124) (end 5.6086 -9.8724) (width 0.25) (layer "F.Cu") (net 6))
 (segment (start 4.9486 -8.340801) (end 4.9486 -9.2124) (width 0.25) (layer "F.Cu") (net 6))
 (segment (start 1.3 -11.6285) (end 1.3232 -11.6517) (width 0.6) (layer "F.Cu") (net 4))
 (segment (start 1.3 -10.89) (end 1.3 -11.6285) (width 0.6) (layer "F.Cu") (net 4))
 (segment (start 1.3232 -12.4968) (end 0.9143 -12.4968) (width 0.6) (layer "F.Cu") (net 4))
 (segment (start 1.3 -11.6285) (end 0.6857 -12.2428) (width 0.6) (layer "F.Cu") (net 4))
 (segment (start 0.9143 -12.4968) (end 0.6857 -12.2682) (width 0.6) (layer "F.Cu") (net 4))
 (segment (start 1.3232 -11.6517) (end 1.3232 -12.4968) (width 0.6) (layer "F.Cu") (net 4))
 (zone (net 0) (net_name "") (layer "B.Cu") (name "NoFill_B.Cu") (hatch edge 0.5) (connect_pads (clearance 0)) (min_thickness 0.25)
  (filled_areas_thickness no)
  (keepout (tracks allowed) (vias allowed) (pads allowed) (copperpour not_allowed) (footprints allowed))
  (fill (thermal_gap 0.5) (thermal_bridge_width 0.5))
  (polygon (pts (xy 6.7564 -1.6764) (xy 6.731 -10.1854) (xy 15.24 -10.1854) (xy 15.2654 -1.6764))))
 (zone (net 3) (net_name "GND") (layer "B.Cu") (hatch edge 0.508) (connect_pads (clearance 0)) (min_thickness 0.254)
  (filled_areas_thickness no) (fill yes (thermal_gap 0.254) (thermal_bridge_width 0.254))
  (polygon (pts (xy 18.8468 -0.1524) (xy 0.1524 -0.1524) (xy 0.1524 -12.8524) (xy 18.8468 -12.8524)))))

